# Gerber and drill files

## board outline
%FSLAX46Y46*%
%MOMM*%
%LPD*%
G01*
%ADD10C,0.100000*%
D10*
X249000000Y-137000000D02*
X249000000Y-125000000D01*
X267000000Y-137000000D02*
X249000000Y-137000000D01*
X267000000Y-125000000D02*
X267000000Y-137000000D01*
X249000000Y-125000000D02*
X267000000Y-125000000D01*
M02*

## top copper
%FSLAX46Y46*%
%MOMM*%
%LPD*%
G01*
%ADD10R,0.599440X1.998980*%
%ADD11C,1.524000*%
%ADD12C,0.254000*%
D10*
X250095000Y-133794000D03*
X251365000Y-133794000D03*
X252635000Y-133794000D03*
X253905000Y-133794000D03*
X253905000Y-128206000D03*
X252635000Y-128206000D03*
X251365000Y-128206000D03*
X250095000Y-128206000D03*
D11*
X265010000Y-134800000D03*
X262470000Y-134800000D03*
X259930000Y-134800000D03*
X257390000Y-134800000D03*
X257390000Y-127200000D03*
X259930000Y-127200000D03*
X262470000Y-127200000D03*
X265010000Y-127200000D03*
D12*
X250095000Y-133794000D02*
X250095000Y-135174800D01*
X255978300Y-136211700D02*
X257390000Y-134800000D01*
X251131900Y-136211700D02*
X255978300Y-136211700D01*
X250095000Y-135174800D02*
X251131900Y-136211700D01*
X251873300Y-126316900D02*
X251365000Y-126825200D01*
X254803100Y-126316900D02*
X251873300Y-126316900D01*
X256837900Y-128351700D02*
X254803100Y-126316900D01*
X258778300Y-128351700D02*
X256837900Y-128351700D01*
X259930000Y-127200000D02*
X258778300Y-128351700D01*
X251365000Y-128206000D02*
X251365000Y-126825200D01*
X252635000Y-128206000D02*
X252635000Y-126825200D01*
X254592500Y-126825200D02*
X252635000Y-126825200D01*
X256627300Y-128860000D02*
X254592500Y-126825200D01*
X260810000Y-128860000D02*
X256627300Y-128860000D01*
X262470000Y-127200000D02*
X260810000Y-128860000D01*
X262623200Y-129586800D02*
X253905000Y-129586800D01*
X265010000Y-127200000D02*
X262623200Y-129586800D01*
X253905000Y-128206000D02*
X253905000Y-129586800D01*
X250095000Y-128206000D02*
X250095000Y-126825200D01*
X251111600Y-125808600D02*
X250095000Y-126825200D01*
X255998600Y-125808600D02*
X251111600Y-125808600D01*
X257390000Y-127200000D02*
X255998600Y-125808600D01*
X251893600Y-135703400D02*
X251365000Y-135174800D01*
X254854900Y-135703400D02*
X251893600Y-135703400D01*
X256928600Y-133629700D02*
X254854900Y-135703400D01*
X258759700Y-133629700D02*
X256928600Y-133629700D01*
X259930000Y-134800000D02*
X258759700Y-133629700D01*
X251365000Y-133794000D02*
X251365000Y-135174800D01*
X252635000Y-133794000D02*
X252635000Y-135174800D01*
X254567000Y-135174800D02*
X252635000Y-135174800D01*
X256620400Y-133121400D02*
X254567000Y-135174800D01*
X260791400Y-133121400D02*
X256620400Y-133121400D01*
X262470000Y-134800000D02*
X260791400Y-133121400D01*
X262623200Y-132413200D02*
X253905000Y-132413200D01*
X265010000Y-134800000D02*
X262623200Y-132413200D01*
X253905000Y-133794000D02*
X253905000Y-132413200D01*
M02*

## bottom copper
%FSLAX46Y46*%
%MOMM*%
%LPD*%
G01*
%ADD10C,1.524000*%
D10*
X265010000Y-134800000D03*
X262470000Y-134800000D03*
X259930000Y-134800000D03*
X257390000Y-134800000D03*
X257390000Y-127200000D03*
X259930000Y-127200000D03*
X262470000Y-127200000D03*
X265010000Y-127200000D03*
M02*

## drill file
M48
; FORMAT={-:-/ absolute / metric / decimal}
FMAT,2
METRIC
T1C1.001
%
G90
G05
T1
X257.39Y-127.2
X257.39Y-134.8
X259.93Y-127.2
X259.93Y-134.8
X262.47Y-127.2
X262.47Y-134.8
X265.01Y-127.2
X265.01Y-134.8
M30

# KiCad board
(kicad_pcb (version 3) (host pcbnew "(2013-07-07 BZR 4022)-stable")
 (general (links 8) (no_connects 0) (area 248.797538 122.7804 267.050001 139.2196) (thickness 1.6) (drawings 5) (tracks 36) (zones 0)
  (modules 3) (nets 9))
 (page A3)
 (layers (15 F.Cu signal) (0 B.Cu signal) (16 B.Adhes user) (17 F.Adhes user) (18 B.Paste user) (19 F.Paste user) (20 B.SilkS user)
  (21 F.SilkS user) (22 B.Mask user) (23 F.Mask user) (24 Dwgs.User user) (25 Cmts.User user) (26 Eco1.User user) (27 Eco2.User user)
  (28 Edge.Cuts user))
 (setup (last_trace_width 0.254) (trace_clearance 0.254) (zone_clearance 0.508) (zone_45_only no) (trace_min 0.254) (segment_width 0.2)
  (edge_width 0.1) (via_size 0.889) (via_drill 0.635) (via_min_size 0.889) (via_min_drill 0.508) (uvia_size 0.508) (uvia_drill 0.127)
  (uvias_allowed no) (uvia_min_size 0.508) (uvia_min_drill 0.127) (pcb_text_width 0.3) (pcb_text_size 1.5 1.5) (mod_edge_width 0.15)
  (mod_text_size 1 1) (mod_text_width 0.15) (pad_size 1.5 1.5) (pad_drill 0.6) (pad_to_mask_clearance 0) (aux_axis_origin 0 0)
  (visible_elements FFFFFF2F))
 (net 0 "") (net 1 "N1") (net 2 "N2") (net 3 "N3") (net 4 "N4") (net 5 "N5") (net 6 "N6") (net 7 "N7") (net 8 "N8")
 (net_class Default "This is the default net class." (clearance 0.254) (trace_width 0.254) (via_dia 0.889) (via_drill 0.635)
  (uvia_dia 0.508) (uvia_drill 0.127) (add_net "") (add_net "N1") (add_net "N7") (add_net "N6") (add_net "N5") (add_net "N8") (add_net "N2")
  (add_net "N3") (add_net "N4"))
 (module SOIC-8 (layer F.Cu) (at 252 131)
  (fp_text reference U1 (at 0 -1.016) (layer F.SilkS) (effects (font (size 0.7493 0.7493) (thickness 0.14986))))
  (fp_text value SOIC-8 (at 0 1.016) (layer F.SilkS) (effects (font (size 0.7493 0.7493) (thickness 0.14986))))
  (pad 1 smd rect (at -1.905 2.794) (size 0.59944 1.99898) (layers F.Cu F.Paste F.Mask) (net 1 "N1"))
  (pad 2 smd rect (at -0.635 2.794) (size 0.59944 1.99898) (layers F.Cu F.Paste F.Mask) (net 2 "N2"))
  (pad 3 smd rect (at 0.635 2.794) (size 0.59944 1.99898) (layers F.Cu F.Paste F.Mask) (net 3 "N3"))
  (pad 4 smd rect (at 1.905 2.794) (size 0.59944 1.99898) (layers F.Cu F.Paste F.Mask) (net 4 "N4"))
  (pad 5 smd rect (at 1.905 -2.794) (size 0.59944 1.99898) (layers F.Cu F.Paste F.Mask) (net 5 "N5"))
  (pad 6 smd rect (at 0.635 -2.794) (size 0.59944 1.99898) (layers F.Cu F.Paste F.Mask) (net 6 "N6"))
  (pad 7 smd rect (at -0.635 -2.794) (size 0.59944 1.99898) (layers F.Cu F.Paste F.Mask) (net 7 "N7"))
  (pad 8 smd rect (at -1.905 -2.794) (size 0.59944 1.99898) (layers F.Cu F.Paste F.Mask) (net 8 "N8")))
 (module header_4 (layer F.Cu) (at 261.2 134.8 180)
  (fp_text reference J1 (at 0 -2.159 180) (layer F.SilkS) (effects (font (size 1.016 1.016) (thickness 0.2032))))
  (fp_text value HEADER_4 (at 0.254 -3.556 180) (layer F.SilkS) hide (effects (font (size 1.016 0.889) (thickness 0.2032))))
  (pad 1 thru_hole circle (at -3.81 0 180) (size 1.524 1.524) (drill 1.00076) (layers *.Cu *.Mask F.SilkS) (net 4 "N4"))
  (pad 2 thru_hole circle (at -1.27 0 180) (size 1.524 2.19964) (drill 1.00076) (layers *.Cu *.Mask F.SilkS) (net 3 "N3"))
  (pad 3 thru_hole circle (at 1.27 0 180) (size 1.524 2.19964) (drill 1.00076) (layers *.Cu *.Mask F.SilkS) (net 2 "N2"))
  (pad 4 thru_hole circle (at 3.81 0 180) (size 1.524 2.19964) (drill 1.00076) (layers *.Cu *.Mask F.SilkS) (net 1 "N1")))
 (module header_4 (layer F.Cu) (at 261.2 127.2)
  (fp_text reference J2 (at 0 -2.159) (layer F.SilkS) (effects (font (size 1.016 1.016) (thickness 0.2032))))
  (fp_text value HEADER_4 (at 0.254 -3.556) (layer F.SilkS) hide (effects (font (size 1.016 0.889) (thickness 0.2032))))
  (pad 1 thru_hole circle (at -3.81 0) (size 1.524 1.524) (drill 1.00076) (layers *.Cu *.Mask F.SilkS) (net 8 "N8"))
  (pad 2 thru_hole circle (at -1.27 0) (size 1.524 2.19964) (drill 1.00076) (layers *.Cu *.Mask F.SilkS) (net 7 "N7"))
  (pad 3 thru_hole circle (at 1.27 0) (size 1.524 2.19964) (drill 1.00076) (layers *.Cu *.Mask F.SilkS) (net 6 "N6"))
  (pad 4 thru_hole circle (at 3.81 0) (size 1.524 2.19964) (drill 1.00076) (layers *.Cu *.Mask F.SilkS) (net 5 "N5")))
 (gr_line (start 249 137) (end 249 125) (angle 90) (layer Edge.Cuts) (width 0.1))
 (gr_line (start 267 137) (end 249 137) (angle 90) (layer Edge.Cuts) (width 0.1))
 (gr_line (start 267 125) (end 267 137) (angle 90) (layer Edge.Cuts) (width 0.1))
 (gr_line (start 249 125) (end 267 125) (angle 90) (layer Edge.Cuts) (width 0.1))
 (segment (start 250.095 133.794) (end 250.095 135.1748) (width 0.254) (layer F.Cu) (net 1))
 (segment (start 255.9783 136.2117) (end 257.39 134.8) (width 0.254) (layer F.Cu) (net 1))
 (segment (start 251.1319 136.2117) (end 255.9783 136.2117) (width 0.254) (layer F.Cu) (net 1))
 (segment (start 250.095 135.1748) (end 251.1319 136.2117) (width 0.254) (layer F.Cu) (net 1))
 (segment (start 251.8733 126.3169) (end 251.365 126.8252) (width 0.254) (layer F.Cu) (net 7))
 (segment (start 254.8031 126.3169) (end 251.8733 126.3169) (width 0.254) (layer F.Cu) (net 7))
 (segment (start 256.8379 128.3517) (end 254.8031 126.3169) (width 0.254) (layer F.Cu) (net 7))
 (segment (start 258.7783 128.3517) (end 256.8379 128.3517) (width 0.254) (layer F.Cu) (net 7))
 (segment (start 259.93 127.2) (end 258.7783 128.3517) (width 0.254) (layer F.Cu) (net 7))
 (segment (start 251.365 128.206) (end 251.365 126.8252) (width 0.254) (layer F.Cu) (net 7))
 (segment (start 252.635 128.206) (end 252.635 126.8252) (width 0.254) (layer F.Cu) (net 6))
 (segment (start 254.5925 126.8252) (end 252.635 126.8252) (width 0.254) (layer F.Cu) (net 6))
 (segment (start 256.6273 128.86) (end 254.5925 126.8252) (width 0.254) (layer F.Cu) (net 6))
 (segment (start 260.81 128.86) (end 256.6273 128.86) (width 0.254) (layer F.Cu) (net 6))
 (segment (start 262.47 127.2) (end 260.81 128.86) (width 0.254) (layer F.Cu) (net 6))
 (segment (start 262.6232 129.5868) (end 253.905 129.5868) (width 0.254) (layer F.Cu) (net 5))
 (segment (start 265.01 127.2) (end 262.6232 129.5868) (width 0.254) (layer F.Cu) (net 5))
 (segment (start 253.905 128.206) (end 253.905 129.5868) (width 0.254) (layer F.Cu) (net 5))
 (segment (start 250.095 128.206) (end 250.095 126.8252) (width 0.254) (layer F.Cu) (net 8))
 (segment (start 251.1116 125.8086) (end 250.095 126.8252) (width 0.254) (layer F.Cu) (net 8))
 (segment (start 255.9986 125.8086) (end 251.1116 125.8086) (width 0.254) (layer F.Cu) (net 8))
 (segment (start 257.39 127.2) (end 255.9986 125.8086) (width 0.254) (layer F.Cu) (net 8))
 (segment (start 251.8936 135.7034) (end 251.365 135.1748) (width 0.254) (layer F.Cu) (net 2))
 (segment (start 254.8549 135.7034) (end 251.8936 135.7034) (width 0.254) (layer F.Cu) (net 2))
 (segment (start 256.9286 133.6297) (end 254.8549 135.7034) (width 0.254) (layer F.Cu) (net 2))
 (segment (start 258.7597 133.6297) (end 256.9286 133.6297) (width 0.254) (layer F.Cu) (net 2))
 (segment (start 259.93 134.8) (end 258.7597 133.6297) (width 0.254) (layer F.Cu) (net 2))
 (segment (start 251.365 133.794) (end 251.365 135.1748) (width 0.254) (layer F.Cu) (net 2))
 (segment (start 252.635 133.794) (end 252.635 135.1748) (width 0.254) (layer F.Cu) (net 3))
 (segment (start 254.567 135.1748) (end 252.635 135.1748) (width 0.254) (layer F.Cu) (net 3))
 (segment (start 256.6204 133.1214) (end 254.567 135.1748) (width 0.254) (layer F.Cu) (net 3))
 (segment (start 260.7914 133.1214) (end 256.6204 133.1214) (width 0.254) (layer F.Cu) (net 3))
 (segment (start 262.47 134.8) (end 260.7914 133.1214) (width 0.254) (layer F.Cu) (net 3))
 (segment (start 262.6232 132.4132) (end 253.905 132.4132) (width 0.254) (layer F.Cu) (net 4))
 (segment (start 265.01 134.8) (end 262.6232 132.4132) (width 0.254) (layer F.Cu) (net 4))
 (segment (start 253.905 133.794) (end 253.905 132.4132) (width 0.254) (layer F.Cu) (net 4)))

